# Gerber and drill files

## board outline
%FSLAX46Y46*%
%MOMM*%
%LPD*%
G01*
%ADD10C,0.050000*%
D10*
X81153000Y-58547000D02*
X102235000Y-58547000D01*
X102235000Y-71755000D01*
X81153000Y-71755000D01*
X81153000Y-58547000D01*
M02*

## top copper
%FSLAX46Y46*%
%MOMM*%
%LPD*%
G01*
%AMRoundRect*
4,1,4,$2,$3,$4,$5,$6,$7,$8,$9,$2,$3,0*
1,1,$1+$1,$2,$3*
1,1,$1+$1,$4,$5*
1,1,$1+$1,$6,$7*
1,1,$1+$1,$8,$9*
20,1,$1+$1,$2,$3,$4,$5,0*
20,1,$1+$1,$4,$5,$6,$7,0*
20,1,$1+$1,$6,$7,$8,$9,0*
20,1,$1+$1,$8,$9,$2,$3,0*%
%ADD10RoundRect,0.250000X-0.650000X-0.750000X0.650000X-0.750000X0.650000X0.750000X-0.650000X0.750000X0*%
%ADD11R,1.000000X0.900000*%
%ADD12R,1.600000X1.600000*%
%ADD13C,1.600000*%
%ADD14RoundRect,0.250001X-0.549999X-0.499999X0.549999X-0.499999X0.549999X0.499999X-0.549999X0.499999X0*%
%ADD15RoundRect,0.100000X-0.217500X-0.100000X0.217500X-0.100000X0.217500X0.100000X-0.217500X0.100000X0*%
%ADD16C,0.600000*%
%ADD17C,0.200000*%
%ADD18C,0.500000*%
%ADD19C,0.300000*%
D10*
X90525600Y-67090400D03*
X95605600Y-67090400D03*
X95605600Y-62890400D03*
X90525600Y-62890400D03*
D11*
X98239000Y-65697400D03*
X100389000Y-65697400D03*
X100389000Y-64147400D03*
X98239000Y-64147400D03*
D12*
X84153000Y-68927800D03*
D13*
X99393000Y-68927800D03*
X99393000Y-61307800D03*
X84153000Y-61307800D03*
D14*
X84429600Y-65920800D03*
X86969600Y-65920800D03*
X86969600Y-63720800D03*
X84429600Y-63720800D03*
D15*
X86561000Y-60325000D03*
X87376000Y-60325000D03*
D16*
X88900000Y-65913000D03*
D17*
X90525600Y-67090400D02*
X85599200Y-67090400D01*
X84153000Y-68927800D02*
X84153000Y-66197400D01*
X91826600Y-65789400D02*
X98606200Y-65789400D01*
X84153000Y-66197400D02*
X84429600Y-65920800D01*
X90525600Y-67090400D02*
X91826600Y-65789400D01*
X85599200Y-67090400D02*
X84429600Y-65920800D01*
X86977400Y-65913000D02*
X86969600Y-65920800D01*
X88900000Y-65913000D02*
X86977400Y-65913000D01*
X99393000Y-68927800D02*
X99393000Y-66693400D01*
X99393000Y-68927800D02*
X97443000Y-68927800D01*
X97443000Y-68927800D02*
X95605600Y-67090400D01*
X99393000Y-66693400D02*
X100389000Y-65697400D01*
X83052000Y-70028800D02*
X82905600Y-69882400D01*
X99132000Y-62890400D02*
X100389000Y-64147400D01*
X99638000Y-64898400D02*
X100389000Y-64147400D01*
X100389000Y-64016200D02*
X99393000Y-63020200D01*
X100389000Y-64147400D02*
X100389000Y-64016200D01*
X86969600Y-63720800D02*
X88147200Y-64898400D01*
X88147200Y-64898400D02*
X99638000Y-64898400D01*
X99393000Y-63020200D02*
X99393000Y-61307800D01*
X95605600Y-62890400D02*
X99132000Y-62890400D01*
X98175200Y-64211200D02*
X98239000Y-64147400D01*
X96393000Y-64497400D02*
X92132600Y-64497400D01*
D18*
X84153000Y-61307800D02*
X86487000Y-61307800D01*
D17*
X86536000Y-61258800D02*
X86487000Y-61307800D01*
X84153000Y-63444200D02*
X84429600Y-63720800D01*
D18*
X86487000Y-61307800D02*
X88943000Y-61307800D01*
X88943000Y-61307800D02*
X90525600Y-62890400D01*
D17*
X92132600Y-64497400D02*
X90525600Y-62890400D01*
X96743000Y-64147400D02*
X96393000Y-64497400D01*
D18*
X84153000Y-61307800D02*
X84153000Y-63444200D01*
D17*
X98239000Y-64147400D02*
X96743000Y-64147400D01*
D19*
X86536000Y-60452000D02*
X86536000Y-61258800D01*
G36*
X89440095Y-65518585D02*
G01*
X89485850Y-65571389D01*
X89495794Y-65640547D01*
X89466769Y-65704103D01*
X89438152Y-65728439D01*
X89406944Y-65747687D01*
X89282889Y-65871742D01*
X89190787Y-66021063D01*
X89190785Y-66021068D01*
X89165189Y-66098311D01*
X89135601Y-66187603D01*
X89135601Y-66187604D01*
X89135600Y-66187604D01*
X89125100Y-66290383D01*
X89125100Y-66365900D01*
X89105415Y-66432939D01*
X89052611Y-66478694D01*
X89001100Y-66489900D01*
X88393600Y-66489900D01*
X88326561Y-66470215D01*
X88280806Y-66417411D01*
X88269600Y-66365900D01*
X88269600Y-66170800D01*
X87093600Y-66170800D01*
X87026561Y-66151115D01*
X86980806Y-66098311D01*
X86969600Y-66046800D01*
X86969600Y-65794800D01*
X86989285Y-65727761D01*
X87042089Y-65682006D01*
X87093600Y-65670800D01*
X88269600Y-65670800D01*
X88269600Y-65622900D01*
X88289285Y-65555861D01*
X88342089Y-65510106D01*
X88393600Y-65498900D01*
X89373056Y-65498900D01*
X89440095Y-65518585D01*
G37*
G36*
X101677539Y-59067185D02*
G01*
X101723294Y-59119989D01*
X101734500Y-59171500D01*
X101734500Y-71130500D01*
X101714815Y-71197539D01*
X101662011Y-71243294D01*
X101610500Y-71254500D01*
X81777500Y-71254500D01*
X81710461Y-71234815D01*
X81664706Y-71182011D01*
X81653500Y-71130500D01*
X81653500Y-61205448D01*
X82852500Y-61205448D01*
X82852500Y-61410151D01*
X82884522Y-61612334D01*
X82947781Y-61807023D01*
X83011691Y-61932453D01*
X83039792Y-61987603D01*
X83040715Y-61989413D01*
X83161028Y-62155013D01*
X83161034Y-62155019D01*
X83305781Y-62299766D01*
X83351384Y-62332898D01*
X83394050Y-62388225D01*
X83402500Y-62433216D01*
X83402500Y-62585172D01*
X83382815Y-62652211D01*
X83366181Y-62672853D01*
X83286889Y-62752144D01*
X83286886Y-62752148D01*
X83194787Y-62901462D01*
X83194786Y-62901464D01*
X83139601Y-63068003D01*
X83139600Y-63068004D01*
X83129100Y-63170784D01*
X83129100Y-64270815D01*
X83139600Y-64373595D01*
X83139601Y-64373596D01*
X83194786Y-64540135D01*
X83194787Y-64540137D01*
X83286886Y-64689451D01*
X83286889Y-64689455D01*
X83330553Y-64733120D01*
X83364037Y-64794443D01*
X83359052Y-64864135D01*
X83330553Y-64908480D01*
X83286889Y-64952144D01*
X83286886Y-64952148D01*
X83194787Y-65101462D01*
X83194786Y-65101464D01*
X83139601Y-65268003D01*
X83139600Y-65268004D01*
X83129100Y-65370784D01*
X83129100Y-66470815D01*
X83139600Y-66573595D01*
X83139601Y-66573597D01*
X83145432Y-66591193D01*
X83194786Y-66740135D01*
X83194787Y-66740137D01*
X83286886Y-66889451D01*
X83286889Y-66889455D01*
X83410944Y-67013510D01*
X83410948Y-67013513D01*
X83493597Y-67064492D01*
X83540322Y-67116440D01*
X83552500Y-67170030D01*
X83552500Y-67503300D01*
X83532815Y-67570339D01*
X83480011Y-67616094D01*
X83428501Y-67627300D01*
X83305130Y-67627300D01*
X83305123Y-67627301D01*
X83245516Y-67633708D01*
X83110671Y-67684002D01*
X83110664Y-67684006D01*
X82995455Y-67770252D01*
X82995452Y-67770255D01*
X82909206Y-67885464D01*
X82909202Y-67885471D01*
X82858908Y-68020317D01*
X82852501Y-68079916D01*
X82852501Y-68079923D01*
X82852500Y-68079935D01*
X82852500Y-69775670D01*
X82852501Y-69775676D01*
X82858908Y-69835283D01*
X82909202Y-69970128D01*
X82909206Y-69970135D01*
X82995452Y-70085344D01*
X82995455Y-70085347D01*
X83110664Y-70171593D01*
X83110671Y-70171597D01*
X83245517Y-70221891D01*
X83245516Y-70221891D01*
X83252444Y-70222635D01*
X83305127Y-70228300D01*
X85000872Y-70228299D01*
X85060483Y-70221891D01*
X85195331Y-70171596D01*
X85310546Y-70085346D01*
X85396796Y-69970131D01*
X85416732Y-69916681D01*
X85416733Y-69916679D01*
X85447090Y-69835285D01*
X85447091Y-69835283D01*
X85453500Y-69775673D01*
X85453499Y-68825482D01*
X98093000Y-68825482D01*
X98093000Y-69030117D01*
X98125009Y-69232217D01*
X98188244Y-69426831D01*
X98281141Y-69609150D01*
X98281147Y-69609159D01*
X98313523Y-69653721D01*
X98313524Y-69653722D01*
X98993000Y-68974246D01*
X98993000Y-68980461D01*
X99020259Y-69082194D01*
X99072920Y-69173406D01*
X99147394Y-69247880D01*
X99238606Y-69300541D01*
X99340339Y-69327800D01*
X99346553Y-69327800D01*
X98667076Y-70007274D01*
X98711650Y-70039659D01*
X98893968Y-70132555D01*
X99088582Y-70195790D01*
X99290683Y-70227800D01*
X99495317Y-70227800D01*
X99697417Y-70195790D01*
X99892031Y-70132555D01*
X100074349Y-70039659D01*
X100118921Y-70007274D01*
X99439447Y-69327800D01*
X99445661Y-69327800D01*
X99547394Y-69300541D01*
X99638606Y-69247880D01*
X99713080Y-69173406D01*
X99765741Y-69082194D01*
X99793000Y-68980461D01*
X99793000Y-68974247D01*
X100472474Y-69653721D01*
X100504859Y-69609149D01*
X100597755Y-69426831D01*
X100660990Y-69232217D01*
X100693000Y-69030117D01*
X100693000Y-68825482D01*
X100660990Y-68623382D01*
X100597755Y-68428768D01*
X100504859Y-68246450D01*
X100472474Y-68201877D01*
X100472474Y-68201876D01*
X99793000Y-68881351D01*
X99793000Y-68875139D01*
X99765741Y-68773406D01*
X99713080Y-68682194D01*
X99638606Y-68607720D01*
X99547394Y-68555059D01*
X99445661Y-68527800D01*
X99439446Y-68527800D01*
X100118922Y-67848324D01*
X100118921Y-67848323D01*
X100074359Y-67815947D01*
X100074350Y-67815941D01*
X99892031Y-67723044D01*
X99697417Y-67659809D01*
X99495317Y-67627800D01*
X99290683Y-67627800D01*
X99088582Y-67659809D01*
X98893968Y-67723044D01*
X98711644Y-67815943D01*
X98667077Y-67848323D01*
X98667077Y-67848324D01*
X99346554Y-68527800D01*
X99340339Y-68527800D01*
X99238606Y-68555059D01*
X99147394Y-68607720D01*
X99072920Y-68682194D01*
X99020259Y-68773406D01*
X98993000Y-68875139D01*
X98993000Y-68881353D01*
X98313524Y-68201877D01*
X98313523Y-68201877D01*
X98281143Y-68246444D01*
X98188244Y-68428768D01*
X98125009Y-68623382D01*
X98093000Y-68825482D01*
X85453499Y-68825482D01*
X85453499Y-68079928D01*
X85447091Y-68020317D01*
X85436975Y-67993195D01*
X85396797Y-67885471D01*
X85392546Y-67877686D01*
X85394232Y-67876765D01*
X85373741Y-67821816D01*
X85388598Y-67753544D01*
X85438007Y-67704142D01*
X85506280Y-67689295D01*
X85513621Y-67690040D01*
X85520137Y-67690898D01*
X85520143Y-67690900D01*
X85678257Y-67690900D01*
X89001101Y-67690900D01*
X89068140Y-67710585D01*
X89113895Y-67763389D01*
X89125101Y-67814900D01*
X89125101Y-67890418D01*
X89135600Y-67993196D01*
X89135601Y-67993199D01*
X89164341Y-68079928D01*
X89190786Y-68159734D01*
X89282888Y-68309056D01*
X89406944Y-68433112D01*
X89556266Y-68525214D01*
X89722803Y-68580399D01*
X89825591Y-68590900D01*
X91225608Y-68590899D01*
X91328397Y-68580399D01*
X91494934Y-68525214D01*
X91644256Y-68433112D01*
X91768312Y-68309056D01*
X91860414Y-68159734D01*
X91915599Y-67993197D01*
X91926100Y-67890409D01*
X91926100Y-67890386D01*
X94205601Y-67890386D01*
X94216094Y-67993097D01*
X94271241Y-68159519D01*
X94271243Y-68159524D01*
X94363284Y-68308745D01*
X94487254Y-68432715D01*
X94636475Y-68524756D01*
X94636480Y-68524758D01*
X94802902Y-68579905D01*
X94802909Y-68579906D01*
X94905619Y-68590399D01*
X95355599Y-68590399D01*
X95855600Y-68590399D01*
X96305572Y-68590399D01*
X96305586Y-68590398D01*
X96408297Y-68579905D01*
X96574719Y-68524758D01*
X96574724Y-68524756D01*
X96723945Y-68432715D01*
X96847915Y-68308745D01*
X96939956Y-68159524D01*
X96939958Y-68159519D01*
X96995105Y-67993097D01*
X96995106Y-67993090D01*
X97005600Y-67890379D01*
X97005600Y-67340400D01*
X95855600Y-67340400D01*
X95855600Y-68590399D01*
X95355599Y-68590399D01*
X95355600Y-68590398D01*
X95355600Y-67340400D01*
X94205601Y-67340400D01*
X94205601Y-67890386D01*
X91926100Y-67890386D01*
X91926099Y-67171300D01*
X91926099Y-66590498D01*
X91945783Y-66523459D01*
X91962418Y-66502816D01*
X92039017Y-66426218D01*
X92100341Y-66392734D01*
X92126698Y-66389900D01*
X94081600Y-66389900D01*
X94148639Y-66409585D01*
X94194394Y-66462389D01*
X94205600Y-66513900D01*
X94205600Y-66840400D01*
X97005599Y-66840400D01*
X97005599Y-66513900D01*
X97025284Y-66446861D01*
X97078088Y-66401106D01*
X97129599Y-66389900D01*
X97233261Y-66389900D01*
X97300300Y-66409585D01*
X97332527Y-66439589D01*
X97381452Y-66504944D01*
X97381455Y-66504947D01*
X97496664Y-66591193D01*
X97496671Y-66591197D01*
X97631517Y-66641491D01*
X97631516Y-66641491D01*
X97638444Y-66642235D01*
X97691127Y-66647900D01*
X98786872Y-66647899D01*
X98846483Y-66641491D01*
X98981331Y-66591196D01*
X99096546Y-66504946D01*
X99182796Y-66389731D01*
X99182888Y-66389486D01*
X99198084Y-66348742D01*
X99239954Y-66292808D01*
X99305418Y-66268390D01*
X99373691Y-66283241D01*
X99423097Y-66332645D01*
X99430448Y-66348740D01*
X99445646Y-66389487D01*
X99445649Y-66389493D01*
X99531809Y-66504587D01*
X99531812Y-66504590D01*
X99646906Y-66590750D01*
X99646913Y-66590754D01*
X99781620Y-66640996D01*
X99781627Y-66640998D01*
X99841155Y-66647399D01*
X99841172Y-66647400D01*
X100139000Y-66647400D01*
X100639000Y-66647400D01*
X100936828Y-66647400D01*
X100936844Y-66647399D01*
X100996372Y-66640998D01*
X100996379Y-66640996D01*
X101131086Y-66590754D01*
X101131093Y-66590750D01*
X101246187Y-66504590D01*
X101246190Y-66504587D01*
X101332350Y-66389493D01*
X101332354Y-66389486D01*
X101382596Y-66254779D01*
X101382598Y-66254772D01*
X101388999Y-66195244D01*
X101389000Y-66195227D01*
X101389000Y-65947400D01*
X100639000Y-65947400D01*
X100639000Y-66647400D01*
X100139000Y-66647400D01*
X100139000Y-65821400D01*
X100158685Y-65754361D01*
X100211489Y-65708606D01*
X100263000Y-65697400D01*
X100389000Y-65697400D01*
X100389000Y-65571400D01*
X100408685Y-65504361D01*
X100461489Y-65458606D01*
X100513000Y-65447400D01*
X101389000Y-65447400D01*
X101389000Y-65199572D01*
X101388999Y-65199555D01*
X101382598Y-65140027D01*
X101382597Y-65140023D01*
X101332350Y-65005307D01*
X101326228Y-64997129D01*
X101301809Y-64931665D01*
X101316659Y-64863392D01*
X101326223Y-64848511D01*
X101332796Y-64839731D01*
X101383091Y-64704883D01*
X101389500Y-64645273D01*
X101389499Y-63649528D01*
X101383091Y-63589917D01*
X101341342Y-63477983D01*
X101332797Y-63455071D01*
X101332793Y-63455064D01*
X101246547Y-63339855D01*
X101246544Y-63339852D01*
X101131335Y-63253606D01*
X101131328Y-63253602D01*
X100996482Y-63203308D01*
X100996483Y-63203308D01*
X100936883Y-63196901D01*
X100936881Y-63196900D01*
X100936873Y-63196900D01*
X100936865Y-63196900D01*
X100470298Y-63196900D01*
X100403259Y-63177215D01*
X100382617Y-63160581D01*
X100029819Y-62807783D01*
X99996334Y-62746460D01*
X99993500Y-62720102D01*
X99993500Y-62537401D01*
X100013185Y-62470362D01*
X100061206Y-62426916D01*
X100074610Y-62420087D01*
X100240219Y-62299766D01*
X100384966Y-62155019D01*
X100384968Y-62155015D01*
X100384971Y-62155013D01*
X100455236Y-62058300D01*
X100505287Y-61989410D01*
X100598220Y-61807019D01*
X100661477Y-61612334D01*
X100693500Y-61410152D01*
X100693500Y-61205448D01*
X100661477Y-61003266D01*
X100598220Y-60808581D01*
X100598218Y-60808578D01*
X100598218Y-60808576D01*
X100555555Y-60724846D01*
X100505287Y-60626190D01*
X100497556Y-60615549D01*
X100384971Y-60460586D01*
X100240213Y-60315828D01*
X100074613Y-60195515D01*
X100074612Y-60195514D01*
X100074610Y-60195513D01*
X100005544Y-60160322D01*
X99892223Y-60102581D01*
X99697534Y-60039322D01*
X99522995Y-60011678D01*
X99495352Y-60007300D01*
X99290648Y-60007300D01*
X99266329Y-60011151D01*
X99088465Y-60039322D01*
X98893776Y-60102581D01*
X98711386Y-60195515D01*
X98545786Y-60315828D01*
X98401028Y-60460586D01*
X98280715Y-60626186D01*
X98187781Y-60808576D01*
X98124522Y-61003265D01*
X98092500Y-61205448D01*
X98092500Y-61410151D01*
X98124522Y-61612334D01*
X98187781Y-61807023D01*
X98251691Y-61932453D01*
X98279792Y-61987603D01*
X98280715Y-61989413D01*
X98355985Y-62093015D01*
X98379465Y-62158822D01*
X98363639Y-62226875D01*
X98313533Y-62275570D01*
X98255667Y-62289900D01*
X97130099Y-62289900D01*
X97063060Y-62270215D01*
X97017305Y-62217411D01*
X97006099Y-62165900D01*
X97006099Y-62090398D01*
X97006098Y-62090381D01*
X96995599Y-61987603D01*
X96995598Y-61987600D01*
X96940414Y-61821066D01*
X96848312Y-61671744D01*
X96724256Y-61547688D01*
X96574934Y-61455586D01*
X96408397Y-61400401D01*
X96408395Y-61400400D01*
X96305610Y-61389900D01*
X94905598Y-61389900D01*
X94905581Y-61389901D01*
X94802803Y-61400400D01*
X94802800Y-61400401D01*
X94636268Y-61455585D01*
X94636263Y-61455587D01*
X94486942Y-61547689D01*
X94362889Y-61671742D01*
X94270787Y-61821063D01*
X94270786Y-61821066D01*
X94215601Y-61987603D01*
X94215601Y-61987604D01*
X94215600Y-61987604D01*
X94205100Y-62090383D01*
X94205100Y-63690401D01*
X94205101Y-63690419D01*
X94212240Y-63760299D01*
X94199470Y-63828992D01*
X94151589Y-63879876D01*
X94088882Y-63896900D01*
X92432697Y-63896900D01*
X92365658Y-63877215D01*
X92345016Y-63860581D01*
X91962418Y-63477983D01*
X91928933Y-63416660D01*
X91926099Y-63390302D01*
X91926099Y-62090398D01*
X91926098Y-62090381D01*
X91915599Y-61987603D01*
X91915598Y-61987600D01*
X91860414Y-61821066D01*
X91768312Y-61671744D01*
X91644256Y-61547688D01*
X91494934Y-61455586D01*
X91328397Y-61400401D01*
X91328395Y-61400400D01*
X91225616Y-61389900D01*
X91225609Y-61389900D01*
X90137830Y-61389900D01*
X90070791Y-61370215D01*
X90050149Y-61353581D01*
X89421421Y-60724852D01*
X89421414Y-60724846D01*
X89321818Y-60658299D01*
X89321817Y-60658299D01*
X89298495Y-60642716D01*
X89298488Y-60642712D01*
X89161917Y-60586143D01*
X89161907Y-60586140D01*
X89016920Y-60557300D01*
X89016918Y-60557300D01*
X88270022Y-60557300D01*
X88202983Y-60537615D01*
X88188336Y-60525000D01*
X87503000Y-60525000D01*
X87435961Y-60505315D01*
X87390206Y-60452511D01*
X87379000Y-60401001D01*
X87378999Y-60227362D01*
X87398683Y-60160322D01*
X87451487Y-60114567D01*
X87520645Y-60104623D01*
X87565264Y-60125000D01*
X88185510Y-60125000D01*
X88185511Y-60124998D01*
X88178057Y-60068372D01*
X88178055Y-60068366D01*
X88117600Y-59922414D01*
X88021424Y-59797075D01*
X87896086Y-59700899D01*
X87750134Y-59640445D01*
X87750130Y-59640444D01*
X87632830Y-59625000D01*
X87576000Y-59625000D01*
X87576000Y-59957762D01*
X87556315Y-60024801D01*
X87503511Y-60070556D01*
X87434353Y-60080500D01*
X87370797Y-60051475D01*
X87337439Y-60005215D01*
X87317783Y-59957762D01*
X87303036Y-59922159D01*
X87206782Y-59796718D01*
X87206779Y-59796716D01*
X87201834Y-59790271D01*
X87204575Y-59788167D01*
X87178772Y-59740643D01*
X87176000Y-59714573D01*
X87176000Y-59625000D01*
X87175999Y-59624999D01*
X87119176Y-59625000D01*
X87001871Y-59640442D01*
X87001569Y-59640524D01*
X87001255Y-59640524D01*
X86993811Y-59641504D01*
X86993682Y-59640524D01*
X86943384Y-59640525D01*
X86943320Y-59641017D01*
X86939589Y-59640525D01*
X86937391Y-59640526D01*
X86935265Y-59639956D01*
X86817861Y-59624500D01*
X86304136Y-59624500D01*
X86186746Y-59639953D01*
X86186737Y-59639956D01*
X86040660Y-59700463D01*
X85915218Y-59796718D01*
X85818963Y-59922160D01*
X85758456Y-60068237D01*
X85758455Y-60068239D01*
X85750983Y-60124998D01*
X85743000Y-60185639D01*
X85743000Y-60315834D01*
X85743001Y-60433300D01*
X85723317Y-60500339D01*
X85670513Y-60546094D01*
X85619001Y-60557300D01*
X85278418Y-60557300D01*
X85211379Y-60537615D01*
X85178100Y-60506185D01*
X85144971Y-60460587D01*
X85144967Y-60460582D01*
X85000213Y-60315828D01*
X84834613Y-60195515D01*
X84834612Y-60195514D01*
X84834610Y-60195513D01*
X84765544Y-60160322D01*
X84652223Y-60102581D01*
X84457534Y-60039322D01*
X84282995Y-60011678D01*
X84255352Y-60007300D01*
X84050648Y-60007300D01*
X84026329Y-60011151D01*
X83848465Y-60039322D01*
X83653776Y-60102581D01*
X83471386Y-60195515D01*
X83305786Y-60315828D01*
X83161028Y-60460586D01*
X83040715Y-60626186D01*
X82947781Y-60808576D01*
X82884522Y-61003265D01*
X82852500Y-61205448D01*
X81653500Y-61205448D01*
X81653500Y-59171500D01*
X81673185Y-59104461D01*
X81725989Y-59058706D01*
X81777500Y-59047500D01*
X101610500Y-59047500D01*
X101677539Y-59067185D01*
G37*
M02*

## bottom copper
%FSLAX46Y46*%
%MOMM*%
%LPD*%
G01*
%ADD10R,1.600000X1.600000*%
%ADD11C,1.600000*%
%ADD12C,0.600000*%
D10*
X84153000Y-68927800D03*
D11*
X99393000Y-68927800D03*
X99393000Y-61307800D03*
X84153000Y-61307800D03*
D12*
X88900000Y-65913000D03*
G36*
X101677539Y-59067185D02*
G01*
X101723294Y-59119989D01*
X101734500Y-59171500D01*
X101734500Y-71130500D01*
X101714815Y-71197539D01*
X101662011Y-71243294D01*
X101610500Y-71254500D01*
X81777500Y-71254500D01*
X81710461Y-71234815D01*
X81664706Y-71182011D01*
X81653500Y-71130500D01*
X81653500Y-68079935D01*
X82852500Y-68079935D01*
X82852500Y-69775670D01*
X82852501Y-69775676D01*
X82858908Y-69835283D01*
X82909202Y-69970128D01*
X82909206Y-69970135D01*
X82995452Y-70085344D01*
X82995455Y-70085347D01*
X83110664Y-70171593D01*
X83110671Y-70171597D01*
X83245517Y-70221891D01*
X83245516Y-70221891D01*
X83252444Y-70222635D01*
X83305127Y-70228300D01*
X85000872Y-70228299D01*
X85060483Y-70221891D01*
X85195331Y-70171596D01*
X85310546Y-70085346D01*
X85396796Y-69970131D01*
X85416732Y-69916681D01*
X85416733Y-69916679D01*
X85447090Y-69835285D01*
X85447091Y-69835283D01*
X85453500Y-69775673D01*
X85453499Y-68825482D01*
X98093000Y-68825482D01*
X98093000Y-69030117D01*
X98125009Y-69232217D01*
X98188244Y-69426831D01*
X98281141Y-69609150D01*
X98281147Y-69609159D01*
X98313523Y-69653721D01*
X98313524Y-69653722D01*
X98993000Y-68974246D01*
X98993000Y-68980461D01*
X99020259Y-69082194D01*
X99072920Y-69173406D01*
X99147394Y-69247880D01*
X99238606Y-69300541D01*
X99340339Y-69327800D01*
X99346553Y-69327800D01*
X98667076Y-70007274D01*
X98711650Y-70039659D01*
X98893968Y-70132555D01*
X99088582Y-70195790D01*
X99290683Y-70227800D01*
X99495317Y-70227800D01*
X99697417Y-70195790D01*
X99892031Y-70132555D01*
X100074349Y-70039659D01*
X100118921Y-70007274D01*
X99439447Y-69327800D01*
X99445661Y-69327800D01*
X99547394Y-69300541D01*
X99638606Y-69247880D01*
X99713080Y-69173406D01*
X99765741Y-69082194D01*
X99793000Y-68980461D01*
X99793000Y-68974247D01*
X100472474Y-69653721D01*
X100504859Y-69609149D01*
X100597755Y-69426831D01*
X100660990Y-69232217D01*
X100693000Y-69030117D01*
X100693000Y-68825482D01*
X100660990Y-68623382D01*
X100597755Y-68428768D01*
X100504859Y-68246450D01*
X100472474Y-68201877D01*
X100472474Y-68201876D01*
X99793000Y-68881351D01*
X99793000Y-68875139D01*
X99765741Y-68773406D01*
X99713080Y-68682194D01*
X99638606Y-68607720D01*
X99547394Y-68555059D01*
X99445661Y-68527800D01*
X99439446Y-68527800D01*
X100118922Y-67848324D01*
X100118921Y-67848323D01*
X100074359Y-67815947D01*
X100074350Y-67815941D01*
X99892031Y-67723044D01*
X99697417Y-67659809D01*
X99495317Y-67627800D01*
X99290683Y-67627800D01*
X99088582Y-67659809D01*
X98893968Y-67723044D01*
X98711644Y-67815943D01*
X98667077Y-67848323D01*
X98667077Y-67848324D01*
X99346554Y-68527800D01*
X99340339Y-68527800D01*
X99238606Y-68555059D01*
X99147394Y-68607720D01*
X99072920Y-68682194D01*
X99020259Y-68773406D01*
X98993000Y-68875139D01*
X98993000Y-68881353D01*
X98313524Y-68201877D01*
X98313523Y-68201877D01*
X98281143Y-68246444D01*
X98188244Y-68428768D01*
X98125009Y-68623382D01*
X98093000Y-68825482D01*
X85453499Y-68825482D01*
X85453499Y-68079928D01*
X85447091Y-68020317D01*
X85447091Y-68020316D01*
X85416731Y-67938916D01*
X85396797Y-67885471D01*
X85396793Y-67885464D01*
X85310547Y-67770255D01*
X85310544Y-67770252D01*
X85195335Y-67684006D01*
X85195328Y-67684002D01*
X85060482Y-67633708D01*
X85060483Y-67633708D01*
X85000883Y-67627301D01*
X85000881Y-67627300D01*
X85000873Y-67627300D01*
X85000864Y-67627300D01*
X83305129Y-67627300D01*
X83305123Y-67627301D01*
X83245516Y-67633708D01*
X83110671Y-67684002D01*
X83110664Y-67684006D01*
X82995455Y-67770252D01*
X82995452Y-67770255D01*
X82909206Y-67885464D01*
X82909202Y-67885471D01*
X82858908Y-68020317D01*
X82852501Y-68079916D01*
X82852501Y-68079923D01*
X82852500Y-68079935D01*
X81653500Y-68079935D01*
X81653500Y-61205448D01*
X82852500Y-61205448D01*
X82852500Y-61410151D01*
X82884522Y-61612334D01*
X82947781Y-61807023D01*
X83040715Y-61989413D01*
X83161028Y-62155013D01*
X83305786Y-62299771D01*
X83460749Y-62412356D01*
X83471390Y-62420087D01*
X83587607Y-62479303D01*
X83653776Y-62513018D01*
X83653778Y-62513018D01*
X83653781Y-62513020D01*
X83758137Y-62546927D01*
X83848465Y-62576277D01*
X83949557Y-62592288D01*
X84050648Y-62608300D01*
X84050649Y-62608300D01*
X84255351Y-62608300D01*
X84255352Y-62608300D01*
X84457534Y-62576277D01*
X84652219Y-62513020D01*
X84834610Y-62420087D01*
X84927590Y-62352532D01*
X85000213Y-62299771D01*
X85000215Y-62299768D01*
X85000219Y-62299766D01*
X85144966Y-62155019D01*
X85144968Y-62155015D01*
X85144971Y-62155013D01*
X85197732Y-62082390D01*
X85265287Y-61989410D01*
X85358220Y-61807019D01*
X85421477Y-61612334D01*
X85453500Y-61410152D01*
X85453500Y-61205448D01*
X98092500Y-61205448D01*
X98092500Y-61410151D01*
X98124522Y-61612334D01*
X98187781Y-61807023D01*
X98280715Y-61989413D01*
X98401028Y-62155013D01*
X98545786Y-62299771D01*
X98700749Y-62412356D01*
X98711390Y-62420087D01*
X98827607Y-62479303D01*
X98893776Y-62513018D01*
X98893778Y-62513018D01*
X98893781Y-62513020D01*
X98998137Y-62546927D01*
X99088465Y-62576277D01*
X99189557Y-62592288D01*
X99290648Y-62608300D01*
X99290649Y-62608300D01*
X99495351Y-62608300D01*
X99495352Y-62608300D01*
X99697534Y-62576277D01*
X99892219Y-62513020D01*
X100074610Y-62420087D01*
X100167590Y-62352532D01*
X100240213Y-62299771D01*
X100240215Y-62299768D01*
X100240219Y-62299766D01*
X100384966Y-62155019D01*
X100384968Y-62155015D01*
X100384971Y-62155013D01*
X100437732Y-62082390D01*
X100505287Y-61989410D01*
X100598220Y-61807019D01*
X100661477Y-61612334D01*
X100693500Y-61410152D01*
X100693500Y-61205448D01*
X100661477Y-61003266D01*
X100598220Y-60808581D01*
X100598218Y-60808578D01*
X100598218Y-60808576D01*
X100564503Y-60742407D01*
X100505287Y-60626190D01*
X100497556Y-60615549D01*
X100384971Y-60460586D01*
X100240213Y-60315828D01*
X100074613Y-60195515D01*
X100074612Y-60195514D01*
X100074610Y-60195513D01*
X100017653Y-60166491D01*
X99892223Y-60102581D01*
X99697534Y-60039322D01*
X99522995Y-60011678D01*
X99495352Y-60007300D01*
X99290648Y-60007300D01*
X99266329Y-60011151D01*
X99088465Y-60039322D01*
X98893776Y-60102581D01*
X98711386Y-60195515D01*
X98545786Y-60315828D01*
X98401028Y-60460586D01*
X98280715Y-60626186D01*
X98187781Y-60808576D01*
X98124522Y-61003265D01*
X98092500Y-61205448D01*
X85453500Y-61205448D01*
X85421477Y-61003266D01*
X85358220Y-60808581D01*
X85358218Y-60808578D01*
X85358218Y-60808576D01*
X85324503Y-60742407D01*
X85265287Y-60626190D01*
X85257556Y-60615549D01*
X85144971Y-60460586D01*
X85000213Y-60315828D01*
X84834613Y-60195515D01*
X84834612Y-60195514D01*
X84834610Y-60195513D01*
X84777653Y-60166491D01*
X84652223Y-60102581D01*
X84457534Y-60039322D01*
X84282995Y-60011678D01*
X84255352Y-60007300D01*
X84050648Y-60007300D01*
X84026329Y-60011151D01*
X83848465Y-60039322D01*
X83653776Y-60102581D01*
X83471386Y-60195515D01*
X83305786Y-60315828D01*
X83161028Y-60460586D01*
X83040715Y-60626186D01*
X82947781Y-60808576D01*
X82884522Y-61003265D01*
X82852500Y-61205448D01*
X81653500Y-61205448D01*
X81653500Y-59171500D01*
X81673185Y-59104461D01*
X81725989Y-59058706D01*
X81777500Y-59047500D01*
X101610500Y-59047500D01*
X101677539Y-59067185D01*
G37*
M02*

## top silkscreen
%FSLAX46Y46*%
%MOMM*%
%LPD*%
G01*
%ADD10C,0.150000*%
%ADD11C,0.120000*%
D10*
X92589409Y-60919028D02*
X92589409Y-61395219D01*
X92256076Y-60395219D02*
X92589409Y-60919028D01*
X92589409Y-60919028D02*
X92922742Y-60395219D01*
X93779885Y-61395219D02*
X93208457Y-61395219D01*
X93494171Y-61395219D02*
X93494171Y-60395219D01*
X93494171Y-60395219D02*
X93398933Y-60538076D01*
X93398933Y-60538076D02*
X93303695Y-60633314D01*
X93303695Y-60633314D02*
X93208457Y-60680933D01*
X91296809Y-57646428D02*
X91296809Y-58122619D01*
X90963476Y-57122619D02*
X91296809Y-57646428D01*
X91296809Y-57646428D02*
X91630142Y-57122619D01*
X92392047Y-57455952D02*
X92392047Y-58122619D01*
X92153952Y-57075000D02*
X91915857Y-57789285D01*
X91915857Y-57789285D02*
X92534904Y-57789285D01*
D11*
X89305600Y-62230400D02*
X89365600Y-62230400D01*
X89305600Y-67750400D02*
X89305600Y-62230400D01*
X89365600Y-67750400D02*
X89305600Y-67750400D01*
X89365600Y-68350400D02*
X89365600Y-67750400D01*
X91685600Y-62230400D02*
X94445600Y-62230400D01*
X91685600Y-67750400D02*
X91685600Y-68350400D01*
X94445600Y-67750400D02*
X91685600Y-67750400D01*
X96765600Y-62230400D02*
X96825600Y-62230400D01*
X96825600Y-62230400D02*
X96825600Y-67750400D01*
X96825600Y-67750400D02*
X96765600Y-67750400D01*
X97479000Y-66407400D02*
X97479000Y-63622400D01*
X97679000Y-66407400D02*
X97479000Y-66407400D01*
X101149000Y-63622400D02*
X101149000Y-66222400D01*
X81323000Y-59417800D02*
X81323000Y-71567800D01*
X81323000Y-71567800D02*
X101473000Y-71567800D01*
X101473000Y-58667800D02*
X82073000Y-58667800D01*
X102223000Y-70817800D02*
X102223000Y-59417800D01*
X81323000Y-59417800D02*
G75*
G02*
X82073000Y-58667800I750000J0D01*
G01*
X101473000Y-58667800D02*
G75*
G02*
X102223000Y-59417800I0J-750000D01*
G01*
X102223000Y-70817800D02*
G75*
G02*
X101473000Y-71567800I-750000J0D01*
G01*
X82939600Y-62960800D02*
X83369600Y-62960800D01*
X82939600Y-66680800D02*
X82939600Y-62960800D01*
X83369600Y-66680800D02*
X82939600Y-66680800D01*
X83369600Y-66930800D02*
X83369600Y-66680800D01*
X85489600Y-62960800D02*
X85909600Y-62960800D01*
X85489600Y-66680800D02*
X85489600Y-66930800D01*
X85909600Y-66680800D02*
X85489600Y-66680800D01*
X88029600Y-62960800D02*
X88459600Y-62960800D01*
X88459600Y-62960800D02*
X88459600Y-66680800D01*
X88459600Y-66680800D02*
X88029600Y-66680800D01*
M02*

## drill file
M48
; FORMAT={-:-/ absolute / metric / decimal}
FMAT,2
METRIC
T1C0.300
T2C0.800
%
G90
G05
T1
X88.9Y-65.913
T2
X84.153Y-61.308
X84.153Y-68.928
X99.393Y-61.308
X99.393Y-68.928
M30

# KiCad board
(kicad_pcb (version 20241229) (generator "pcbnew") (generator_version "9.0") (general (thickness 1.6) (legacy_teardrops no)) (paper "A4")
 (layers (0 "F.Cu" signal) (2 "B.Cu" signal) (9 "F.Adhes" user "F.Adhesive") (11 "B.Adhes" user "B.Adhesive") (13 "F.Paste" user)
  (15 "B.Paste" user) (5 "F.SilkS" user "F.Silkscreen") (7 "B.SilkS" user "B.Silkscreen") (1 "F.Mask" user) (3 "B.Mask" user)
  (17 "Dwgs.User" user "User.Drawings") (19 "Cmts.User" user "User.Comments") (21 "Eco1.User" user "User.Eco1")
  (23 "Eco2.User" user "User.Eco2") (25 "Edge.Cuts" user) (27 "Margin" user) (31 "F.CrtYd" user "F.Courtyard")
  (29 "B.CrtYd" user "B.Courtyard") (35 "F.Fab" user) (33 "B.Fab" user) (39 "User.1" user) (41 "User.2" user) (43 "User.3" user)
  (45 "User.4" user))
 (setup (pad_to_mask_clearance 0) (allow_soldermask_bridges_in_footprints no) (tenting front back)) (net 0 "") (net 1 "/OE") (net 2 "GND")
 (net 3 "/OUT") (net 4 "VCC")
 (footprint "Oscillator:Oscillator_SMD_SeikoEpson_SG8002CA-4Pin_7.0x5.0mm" (layer "F.Cu") (at 93.0656 64.9904)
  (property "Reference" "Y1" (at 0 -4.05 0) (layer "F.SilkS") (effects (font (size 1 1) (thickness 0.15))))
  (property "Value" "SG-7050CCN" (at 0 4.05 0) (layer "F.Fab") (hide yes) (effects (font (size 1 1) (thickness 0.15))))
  (fp_line (start -3.76 -2.76) (end -3.7 -2.76) (stroke (width 0.12) (type solid)) (layer "F.SilkS"))
  (fp_line (start -3.76 2.76) (end -3.76 -2.76) (stroke (width 0.12) (type solid)) (layer "F.SilkS"))
  (fp_line (start -3.7 2.76) (end -3.76 2.76) (stroke (width 0.12) (type solid)) (layer "F.SilkS"))
  (fp_line (start -3.7 3.36) (end -3.7 2.76) (stroke (width 0.12) (type solid)) (layer "F.SilkS"))
  (fp_line (start -1.38 -2.76) (end 1.38 -2.76) (stroke (width 0.12) (type solid)) (layer "F.SilkS"))
  (fp_line (start -1.38 2.76) (end -1.38 3.36) (stroke (width 0.12) (type solid)) (layer "F.SilkS"))
  (fp_line (start 1.38 2.76) (end -1.38 2.76) (stroke (width 0.12) (type solid)) (layer "F.SilkS"))
  (fp_line (start 3.7 -2.76) (end 3.76 -2.76) (stroke (width 0.12) (type solid)) (layer "F.SilkS"))
  (fp_line (start 3.76 -2.76) (end 3.76 2.76) (stroke (width 0.12) (type solid)) (layer "F.SilkS"))
  (fp_line (start 3.76 2.76) (end 3.7 2.76) (stroke (width 0.12) (type solid)) (layer "F.SilkS"))
  (pad "1" smd roundrect (at -2.54 2.1) (size 1.8 2) (layers "F.Cu" "F.Mask" "F.Paste") (roundrect_rratio 0.138889) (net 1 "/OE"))
  (pad "2" smd roundrect (at 2.54 2.1) (size 1.8 2) (layers "F.Cu" "F.Mask" "F.Paste") (roundrect_rratio 0.138889) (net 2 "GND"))
  (pad "3" smd roundrect (at 2.54 -2.1) (size 1.8 2) (layers "F.Cu" "F.Mask" "F.Paste") (roundrect_rratio 0.138889) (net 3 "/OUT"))
  (pad "4" smd roundrect (at -2.54 -2.1) (size 1.8 2) (layers "F.Cu" "F.Mask" "F.Paste") (roundrect_rratio 0.138889) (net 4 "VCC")))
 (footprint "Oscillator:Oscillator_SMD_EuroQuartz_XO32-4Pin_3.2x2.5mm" (layer "F.Cu") (at 99.314 64.9224 90)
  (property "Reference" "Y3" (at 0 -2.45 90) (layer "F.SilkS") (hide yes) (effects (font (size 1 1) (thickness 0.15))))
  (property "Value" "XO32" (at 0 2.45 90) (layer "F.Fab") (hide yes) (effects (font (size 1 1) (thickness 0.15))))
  (fp_line (start -1.485 -1.835) (end 1.3 -1.835) (stroke (width 0.12) (type solid)) (layer "F.SilkS"))
  (fp_line (start -1.485 -1.635) (end -1.485 -1.835) (stroke (width 0.12) (type solid)) (layer "F.SilkS"))
  (fp_line (start 1.3 1.835) (end -1.3 1.835) (stroke (width 0.12) (type solid)) (layer "F.SilkS"))
  (pad "1" smd rect (at -0.775 -1.075) (size 1 0.9) (layers "F.Cu" "F.Mask" "F.Paste") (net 1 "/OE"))
  (pad "2" smd rect (at -0.775 1.075) (size 1 0.9) (layers "F.Cu" "F.Mask" "F.Paste") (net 2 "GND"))
  (pad "3" smd rect (at 0.775 1.075) (size 1 0.9) (layers "F.Cu" "F.Mask" "F.Paste") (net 3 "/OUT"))
  (pad "4" smd rect (at 0.775 -1.075) (size 1 0.9) (layers "F.Cu" "F.Mask" "F.Paste") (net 4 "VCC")))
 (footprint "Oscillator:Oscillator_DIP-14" (layer "F.Cu") (at 84.153 68.9278)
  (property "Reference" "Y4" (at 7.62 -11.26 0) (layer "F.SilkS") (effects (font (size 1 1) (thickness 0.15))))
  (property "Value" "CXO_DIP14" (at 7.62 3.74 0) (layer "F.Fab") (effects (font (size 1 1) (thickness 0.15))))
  (fp_line (start -2.83 -9.51) (end -2.83 2.64) (stroke (width 0.12) (type solid)) (layer "F.SilkS"))
  (fp_line (start -2.83 2.64) (end 17.32 2.64) (stroke (width 0.12) (type solid)) (layer "F.SilkS"))
  (fp_line (start 17.32 -10.26) (end -2.08 -10.26) (stroke (width 0.12) (type solid)) (layer "F.SilkS"))
  (fp_line (start 18.07 1.89) (end 18.07 -9.51) (stroke (width 0.12) (type solid)) (layer "F.SilkS"))
  (fp_arc (start -2.83 -9.51) (mid -2.61033 -10.04033) (end -2.08 -10.26) (stroke (width 0.12) (type solid)) (layer "F.SilkS"))
  (fp_arc (start 17.32 -10.26) (mid 17.85033 -10.04033) (end 18.07 -9.51) (stroke (width 0.12) (type solid)) (layer "F.SilkS"))
  (fp_arc (start 18.07 1.89) (mid 17.85033 2.42033) (end 17.32 2.64) (stroke (width 0.12) (type solid)) (layer "F.SilkS"))
  (pad "1" thru_hole rect (at 0 0) (size 1.6 1.6) (drill 0.8) (layers "*.Cu" "*.Mask") (remove_unused_layers no) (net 1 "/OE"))
  (pad "7" thru_hole circle (at 15.24 0) (size 1.6 1.6) (drill 0.8) (layers "*.Cu" "*.Mask") (remove_unused_layers no) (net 2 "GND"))
  (pad "8" thru_hole circle (at 15.24 -7.62) (size 1.6 1.6) (drill 0.8) (layers "*.Cu" "*.Mask") (remove_unused_layers no) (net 3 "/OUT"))
  (pad "14" thru_hole circle (at 0 -7.62) (size 1.6 1.6) (drill 0.8) (layers "*.Cu" "*.Mask") (remove_unused_layers no) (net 4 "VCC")))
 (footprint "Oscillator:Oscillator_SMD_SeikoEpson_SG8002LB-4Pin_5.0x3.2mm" (layer "F.Cu") (at 85.6996 64.8208)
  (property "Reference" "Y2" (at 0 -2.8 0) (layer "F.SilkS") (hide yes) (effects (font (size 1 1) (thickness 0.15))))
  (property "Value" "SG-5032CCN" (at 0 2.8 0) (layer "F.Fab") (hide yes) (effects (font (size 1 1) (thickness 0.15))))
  (fp_line (start -2.76 -1.86) (end -2.33 -1.86) (stroke (width 0.12) (type solid)) (layer "F.SilkS"))
  (fp_line (start -2.76 1.86) (end -2.76 -1.86) (stroke (width 0.12) (type solid)) (layer "F.SilkS"))
  (fp_line (start -2.33 1.86) (end -2.76 1.86) (stroke (width 0.12) (type solid)) (layer "F.SilkS"))
  (fp_line (start -2.33 2.11) (end -2.33 1.86) (stroke (width 0.12) (type solid)) (layer "F.SilkS"))
  (fp_line (start -0.21 -1.86) (end 0.21 -1.86) (stroke (width 0.12) (type solid)) (layer "F.SilkS"))
  (fp_line (start -0.21 1.86) (end -0.21 2.11) (stroke (width 0.12) (type solid)) (layer "F.SilkS"))
  (fp_line (start 0.21 1.86) (end -0.21 1.86) (stroke (width 0.12) (type solid)) (layer "F.SilkS"))
  (fp_line (start 2.33 -1.86) (end 2.76 -1.86) (stroke (width 0.12) (type solid)) (layer "F.SilkS"))
  (fp_line (start 2.76 -1.86) (end 2.76 1.86) (stroke (width 0.12) (type solid)) (layer "F.SilkS"))
  (fp_line (start 2.76 1.86) (end 2.33 1.86) (stroke (width 0.12) (type solid)) (layer "F.SilkS"))
  (pad "1" smd roundrect (at -1.27 1.1) (size 1.6 1.5) (layers "F.Cu" "F.Mask" "F.Paste") (roundrect_rratio 0.166667) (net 1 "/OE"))
  (pad "2" smd roundrect (at 1.27 1.1) (size 1.6 1.5) (layers "F.Cu" "F.Mask" "F.Paste") (roundrect_rratio 0.166667) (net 2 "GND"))
  (pad "3" smd roundrect (at 1.27 -1.1) (size 1.6 1.5) (layers "F.Cu" "F.Mask" "F.Paste") (roundrect_rratio 0.166667) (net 3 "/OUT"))
  (pad "4" smd roundrect (at -1.27 -1.1) (size 1.6 1.5) (layers "F.Cu" "F.Mask" "F.Paste") (roundrect_rratio 0.166667) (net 4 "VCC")))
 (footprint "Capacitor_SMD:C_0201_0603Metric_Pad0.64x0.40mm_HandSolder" (layer "F.Cu") (at 86.9685 60.325)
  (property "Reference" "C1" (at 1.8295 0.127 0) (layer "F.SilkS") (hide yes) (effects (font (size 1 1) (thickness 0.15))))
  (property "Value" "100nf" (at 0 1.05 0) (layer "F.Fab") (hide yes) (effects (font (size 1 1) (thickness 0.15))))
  (pad "" smd roundrect (at -0.4325 0) (size 0.458 0.36) (layers "F.Paste") (roundrect_rratio 0.25))
  (pad "" smd roundrect (at 0.4325 0) (size 0.458 0.36) (layers "F.Paste") (roundrect_rratio 0.25))
  (pad "1" smd roundrect (at -0.4075 0) (size 0.635 0.4) (layers "F.Cu" "F.Mask") (roundrect_rratio 0.25) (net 4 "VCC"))
  (pad "2" smd roundrect (at 0.4075 0) (size 0.635 0.4) (layers "F.Cu" "F.Mask") (roundrect_rratio 0.25) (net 2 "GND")))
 (gr_rect (start 81.153 58.547) (end 102.235 71.755) (stroke (width 0.05) (type default)) (fill no) (layer "Edge.Cuts"))
 (segment (start 90.5256 67.0904) (end 85.5992 67.0904) (width 0.2) (layer "F.Cu") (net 1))
 (segment (start 84.153 68.9278) (end 84.153 66.1974) (width 0.2) (layer "F.Cu") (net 1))
 (segment (start 91.8266 65.7894) (end 98.6062 65.7894) (width 0.2) (layer "F.Cu") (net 1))
 (segment (start 84.153 66.1974) (end 84.4296 65.9208) (width 0.2) (layer "F.Cu") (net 1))
 (segment (start 90.5256 67.0904) (end 91.8266 65.7894) (width 0.2) (layer "F.Cu") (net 1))
 (segment (start 85.5992 67.0904) (end 84.4296 65.9208) (width 0.2) (layer "F.Cu") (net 1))
 (segment (start 86.9774 65.913) (end 86.9696 65.9208) (width 0.2) (layer "F.Cu") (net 2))
 (segment (start 88.9 65.913) (end 86.9774 65.913) (width 0.2) (layer "F.Cu") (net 2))
 (segment (start 99.393 68.9278) (end 99.393 66.6934) (width 0.2) (layer "F.Cu") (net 2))
 (segment (start 99.393 68.9278) (end 97.443 68.9278) (width 0.2) (layer "F.Cu") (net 2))
 (segment (start 97.443 68.9278) (end 95.6056 67.0904) (width 0.2) (layer "F.Cu") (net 2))
 (segment (start 99.393 66.6934) (end 100.389 65.6974) (width 0.2) (layer "F.Cu") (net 2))
 (segment (start 83.052 70.0288) (end 82.9056 69.8824) (width 0.2) (layer "F.Cu") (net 2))
 (via (at 88.9 65.913) (size 0.6) (drill 0.3) (layers "F.Cu" "B.Cu") (free yes) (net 2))
 (segment (start 99.132 62.8904) (end 100.389 64.1474) (width 0.2) (layer "F.Cu") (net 3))
 (segment (start 99.638 64.8984) (end 100.389 64.1474) (width 0.2) (layer "F.Cu") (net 3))
 (segment (start 100.389 64.0162) (end 99.393 63.0202) (width 0.2) (layer "F.Cu") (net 3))
 (segment (start 100.389 64.1474) (end 100.389 64.0162) (width 0.2) (layer "F.Cu") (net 3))
 (segment (start 86.9696 63.7208) (end 88.1472 64.8984) (width 0.2) (layer "F.Cu") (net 3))
 (segment (start 88.1472 64.8984) (end 99.638 64.8984) (width 0.2) (layer "F.Cu") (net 3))
 (segment (start 99.393 63.0202) (end 99.393 61.3078) (width 0.2) (layer "F.Cu") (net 3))
 (segment (start 95.6056 62.8904) (end 99.132 62.8904) (width 0.2) (layer "F.Cu") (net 3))
 (segment (start 98.1752 64.2112) (end 98.239 64.1474) (width 0.2) (layer "F.Cu") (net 4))
 (segment (start 96.393 64.4974) (end 92.1326 64.4974) (width 0.2) (layer "F.Cu") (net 4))
 (segment (start 84.153 61.3078) (end 86.487 61.3078) (width 0.5) (layer "F.Cu") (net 4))
 (segment (start 86.536 61.2588) (end 86.487 61.3078) (width 0.2) (layer "F.Cu") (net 4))
 (segment (start 84.153 63.4442) (end 84.4296 63.7208) (width 0.2) (layer "F.Cu") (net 4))
 (segment (start 86.487 61.3078) (end 88.943 61.3078) (width 0.5) (layer "F.Cu") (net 4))
 (segment (start 88.943 61.3078) (end 90.5256 62.8904) (width 0.5) (layer "F.Cu") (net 4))
 (segment (start 92.1326 64.4974) (end 90.5256 62.8904) (width 0.2) (layer "F.Cu") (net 4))
 (segment (start 96.743 64.1474) (end 96.393 64.4974) (width 0.2) (layer "F.Cu") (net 4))
 (segment (start 84.153 61.3078) (end 84.153 63.4442) (width 0.5) (layer "F.Cu") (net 4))
 (segment (start 98.239 64.1474) (end 96.743 64.1474) (width 0.2) (layer "F.Cu") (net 4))
 (segment (start 86.536 60.452) (end 86.536 61.2588) (width 0.3) (layer "F.Cu") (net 4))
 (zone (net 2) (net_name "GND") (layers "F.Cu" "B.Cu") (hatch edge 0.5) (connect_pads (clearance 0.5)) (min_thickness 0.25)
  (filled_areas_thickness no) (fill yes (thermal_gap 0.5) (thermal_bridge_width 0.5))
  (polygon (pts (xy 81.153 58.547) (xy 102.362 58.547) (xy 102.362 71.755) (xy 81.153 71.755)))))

